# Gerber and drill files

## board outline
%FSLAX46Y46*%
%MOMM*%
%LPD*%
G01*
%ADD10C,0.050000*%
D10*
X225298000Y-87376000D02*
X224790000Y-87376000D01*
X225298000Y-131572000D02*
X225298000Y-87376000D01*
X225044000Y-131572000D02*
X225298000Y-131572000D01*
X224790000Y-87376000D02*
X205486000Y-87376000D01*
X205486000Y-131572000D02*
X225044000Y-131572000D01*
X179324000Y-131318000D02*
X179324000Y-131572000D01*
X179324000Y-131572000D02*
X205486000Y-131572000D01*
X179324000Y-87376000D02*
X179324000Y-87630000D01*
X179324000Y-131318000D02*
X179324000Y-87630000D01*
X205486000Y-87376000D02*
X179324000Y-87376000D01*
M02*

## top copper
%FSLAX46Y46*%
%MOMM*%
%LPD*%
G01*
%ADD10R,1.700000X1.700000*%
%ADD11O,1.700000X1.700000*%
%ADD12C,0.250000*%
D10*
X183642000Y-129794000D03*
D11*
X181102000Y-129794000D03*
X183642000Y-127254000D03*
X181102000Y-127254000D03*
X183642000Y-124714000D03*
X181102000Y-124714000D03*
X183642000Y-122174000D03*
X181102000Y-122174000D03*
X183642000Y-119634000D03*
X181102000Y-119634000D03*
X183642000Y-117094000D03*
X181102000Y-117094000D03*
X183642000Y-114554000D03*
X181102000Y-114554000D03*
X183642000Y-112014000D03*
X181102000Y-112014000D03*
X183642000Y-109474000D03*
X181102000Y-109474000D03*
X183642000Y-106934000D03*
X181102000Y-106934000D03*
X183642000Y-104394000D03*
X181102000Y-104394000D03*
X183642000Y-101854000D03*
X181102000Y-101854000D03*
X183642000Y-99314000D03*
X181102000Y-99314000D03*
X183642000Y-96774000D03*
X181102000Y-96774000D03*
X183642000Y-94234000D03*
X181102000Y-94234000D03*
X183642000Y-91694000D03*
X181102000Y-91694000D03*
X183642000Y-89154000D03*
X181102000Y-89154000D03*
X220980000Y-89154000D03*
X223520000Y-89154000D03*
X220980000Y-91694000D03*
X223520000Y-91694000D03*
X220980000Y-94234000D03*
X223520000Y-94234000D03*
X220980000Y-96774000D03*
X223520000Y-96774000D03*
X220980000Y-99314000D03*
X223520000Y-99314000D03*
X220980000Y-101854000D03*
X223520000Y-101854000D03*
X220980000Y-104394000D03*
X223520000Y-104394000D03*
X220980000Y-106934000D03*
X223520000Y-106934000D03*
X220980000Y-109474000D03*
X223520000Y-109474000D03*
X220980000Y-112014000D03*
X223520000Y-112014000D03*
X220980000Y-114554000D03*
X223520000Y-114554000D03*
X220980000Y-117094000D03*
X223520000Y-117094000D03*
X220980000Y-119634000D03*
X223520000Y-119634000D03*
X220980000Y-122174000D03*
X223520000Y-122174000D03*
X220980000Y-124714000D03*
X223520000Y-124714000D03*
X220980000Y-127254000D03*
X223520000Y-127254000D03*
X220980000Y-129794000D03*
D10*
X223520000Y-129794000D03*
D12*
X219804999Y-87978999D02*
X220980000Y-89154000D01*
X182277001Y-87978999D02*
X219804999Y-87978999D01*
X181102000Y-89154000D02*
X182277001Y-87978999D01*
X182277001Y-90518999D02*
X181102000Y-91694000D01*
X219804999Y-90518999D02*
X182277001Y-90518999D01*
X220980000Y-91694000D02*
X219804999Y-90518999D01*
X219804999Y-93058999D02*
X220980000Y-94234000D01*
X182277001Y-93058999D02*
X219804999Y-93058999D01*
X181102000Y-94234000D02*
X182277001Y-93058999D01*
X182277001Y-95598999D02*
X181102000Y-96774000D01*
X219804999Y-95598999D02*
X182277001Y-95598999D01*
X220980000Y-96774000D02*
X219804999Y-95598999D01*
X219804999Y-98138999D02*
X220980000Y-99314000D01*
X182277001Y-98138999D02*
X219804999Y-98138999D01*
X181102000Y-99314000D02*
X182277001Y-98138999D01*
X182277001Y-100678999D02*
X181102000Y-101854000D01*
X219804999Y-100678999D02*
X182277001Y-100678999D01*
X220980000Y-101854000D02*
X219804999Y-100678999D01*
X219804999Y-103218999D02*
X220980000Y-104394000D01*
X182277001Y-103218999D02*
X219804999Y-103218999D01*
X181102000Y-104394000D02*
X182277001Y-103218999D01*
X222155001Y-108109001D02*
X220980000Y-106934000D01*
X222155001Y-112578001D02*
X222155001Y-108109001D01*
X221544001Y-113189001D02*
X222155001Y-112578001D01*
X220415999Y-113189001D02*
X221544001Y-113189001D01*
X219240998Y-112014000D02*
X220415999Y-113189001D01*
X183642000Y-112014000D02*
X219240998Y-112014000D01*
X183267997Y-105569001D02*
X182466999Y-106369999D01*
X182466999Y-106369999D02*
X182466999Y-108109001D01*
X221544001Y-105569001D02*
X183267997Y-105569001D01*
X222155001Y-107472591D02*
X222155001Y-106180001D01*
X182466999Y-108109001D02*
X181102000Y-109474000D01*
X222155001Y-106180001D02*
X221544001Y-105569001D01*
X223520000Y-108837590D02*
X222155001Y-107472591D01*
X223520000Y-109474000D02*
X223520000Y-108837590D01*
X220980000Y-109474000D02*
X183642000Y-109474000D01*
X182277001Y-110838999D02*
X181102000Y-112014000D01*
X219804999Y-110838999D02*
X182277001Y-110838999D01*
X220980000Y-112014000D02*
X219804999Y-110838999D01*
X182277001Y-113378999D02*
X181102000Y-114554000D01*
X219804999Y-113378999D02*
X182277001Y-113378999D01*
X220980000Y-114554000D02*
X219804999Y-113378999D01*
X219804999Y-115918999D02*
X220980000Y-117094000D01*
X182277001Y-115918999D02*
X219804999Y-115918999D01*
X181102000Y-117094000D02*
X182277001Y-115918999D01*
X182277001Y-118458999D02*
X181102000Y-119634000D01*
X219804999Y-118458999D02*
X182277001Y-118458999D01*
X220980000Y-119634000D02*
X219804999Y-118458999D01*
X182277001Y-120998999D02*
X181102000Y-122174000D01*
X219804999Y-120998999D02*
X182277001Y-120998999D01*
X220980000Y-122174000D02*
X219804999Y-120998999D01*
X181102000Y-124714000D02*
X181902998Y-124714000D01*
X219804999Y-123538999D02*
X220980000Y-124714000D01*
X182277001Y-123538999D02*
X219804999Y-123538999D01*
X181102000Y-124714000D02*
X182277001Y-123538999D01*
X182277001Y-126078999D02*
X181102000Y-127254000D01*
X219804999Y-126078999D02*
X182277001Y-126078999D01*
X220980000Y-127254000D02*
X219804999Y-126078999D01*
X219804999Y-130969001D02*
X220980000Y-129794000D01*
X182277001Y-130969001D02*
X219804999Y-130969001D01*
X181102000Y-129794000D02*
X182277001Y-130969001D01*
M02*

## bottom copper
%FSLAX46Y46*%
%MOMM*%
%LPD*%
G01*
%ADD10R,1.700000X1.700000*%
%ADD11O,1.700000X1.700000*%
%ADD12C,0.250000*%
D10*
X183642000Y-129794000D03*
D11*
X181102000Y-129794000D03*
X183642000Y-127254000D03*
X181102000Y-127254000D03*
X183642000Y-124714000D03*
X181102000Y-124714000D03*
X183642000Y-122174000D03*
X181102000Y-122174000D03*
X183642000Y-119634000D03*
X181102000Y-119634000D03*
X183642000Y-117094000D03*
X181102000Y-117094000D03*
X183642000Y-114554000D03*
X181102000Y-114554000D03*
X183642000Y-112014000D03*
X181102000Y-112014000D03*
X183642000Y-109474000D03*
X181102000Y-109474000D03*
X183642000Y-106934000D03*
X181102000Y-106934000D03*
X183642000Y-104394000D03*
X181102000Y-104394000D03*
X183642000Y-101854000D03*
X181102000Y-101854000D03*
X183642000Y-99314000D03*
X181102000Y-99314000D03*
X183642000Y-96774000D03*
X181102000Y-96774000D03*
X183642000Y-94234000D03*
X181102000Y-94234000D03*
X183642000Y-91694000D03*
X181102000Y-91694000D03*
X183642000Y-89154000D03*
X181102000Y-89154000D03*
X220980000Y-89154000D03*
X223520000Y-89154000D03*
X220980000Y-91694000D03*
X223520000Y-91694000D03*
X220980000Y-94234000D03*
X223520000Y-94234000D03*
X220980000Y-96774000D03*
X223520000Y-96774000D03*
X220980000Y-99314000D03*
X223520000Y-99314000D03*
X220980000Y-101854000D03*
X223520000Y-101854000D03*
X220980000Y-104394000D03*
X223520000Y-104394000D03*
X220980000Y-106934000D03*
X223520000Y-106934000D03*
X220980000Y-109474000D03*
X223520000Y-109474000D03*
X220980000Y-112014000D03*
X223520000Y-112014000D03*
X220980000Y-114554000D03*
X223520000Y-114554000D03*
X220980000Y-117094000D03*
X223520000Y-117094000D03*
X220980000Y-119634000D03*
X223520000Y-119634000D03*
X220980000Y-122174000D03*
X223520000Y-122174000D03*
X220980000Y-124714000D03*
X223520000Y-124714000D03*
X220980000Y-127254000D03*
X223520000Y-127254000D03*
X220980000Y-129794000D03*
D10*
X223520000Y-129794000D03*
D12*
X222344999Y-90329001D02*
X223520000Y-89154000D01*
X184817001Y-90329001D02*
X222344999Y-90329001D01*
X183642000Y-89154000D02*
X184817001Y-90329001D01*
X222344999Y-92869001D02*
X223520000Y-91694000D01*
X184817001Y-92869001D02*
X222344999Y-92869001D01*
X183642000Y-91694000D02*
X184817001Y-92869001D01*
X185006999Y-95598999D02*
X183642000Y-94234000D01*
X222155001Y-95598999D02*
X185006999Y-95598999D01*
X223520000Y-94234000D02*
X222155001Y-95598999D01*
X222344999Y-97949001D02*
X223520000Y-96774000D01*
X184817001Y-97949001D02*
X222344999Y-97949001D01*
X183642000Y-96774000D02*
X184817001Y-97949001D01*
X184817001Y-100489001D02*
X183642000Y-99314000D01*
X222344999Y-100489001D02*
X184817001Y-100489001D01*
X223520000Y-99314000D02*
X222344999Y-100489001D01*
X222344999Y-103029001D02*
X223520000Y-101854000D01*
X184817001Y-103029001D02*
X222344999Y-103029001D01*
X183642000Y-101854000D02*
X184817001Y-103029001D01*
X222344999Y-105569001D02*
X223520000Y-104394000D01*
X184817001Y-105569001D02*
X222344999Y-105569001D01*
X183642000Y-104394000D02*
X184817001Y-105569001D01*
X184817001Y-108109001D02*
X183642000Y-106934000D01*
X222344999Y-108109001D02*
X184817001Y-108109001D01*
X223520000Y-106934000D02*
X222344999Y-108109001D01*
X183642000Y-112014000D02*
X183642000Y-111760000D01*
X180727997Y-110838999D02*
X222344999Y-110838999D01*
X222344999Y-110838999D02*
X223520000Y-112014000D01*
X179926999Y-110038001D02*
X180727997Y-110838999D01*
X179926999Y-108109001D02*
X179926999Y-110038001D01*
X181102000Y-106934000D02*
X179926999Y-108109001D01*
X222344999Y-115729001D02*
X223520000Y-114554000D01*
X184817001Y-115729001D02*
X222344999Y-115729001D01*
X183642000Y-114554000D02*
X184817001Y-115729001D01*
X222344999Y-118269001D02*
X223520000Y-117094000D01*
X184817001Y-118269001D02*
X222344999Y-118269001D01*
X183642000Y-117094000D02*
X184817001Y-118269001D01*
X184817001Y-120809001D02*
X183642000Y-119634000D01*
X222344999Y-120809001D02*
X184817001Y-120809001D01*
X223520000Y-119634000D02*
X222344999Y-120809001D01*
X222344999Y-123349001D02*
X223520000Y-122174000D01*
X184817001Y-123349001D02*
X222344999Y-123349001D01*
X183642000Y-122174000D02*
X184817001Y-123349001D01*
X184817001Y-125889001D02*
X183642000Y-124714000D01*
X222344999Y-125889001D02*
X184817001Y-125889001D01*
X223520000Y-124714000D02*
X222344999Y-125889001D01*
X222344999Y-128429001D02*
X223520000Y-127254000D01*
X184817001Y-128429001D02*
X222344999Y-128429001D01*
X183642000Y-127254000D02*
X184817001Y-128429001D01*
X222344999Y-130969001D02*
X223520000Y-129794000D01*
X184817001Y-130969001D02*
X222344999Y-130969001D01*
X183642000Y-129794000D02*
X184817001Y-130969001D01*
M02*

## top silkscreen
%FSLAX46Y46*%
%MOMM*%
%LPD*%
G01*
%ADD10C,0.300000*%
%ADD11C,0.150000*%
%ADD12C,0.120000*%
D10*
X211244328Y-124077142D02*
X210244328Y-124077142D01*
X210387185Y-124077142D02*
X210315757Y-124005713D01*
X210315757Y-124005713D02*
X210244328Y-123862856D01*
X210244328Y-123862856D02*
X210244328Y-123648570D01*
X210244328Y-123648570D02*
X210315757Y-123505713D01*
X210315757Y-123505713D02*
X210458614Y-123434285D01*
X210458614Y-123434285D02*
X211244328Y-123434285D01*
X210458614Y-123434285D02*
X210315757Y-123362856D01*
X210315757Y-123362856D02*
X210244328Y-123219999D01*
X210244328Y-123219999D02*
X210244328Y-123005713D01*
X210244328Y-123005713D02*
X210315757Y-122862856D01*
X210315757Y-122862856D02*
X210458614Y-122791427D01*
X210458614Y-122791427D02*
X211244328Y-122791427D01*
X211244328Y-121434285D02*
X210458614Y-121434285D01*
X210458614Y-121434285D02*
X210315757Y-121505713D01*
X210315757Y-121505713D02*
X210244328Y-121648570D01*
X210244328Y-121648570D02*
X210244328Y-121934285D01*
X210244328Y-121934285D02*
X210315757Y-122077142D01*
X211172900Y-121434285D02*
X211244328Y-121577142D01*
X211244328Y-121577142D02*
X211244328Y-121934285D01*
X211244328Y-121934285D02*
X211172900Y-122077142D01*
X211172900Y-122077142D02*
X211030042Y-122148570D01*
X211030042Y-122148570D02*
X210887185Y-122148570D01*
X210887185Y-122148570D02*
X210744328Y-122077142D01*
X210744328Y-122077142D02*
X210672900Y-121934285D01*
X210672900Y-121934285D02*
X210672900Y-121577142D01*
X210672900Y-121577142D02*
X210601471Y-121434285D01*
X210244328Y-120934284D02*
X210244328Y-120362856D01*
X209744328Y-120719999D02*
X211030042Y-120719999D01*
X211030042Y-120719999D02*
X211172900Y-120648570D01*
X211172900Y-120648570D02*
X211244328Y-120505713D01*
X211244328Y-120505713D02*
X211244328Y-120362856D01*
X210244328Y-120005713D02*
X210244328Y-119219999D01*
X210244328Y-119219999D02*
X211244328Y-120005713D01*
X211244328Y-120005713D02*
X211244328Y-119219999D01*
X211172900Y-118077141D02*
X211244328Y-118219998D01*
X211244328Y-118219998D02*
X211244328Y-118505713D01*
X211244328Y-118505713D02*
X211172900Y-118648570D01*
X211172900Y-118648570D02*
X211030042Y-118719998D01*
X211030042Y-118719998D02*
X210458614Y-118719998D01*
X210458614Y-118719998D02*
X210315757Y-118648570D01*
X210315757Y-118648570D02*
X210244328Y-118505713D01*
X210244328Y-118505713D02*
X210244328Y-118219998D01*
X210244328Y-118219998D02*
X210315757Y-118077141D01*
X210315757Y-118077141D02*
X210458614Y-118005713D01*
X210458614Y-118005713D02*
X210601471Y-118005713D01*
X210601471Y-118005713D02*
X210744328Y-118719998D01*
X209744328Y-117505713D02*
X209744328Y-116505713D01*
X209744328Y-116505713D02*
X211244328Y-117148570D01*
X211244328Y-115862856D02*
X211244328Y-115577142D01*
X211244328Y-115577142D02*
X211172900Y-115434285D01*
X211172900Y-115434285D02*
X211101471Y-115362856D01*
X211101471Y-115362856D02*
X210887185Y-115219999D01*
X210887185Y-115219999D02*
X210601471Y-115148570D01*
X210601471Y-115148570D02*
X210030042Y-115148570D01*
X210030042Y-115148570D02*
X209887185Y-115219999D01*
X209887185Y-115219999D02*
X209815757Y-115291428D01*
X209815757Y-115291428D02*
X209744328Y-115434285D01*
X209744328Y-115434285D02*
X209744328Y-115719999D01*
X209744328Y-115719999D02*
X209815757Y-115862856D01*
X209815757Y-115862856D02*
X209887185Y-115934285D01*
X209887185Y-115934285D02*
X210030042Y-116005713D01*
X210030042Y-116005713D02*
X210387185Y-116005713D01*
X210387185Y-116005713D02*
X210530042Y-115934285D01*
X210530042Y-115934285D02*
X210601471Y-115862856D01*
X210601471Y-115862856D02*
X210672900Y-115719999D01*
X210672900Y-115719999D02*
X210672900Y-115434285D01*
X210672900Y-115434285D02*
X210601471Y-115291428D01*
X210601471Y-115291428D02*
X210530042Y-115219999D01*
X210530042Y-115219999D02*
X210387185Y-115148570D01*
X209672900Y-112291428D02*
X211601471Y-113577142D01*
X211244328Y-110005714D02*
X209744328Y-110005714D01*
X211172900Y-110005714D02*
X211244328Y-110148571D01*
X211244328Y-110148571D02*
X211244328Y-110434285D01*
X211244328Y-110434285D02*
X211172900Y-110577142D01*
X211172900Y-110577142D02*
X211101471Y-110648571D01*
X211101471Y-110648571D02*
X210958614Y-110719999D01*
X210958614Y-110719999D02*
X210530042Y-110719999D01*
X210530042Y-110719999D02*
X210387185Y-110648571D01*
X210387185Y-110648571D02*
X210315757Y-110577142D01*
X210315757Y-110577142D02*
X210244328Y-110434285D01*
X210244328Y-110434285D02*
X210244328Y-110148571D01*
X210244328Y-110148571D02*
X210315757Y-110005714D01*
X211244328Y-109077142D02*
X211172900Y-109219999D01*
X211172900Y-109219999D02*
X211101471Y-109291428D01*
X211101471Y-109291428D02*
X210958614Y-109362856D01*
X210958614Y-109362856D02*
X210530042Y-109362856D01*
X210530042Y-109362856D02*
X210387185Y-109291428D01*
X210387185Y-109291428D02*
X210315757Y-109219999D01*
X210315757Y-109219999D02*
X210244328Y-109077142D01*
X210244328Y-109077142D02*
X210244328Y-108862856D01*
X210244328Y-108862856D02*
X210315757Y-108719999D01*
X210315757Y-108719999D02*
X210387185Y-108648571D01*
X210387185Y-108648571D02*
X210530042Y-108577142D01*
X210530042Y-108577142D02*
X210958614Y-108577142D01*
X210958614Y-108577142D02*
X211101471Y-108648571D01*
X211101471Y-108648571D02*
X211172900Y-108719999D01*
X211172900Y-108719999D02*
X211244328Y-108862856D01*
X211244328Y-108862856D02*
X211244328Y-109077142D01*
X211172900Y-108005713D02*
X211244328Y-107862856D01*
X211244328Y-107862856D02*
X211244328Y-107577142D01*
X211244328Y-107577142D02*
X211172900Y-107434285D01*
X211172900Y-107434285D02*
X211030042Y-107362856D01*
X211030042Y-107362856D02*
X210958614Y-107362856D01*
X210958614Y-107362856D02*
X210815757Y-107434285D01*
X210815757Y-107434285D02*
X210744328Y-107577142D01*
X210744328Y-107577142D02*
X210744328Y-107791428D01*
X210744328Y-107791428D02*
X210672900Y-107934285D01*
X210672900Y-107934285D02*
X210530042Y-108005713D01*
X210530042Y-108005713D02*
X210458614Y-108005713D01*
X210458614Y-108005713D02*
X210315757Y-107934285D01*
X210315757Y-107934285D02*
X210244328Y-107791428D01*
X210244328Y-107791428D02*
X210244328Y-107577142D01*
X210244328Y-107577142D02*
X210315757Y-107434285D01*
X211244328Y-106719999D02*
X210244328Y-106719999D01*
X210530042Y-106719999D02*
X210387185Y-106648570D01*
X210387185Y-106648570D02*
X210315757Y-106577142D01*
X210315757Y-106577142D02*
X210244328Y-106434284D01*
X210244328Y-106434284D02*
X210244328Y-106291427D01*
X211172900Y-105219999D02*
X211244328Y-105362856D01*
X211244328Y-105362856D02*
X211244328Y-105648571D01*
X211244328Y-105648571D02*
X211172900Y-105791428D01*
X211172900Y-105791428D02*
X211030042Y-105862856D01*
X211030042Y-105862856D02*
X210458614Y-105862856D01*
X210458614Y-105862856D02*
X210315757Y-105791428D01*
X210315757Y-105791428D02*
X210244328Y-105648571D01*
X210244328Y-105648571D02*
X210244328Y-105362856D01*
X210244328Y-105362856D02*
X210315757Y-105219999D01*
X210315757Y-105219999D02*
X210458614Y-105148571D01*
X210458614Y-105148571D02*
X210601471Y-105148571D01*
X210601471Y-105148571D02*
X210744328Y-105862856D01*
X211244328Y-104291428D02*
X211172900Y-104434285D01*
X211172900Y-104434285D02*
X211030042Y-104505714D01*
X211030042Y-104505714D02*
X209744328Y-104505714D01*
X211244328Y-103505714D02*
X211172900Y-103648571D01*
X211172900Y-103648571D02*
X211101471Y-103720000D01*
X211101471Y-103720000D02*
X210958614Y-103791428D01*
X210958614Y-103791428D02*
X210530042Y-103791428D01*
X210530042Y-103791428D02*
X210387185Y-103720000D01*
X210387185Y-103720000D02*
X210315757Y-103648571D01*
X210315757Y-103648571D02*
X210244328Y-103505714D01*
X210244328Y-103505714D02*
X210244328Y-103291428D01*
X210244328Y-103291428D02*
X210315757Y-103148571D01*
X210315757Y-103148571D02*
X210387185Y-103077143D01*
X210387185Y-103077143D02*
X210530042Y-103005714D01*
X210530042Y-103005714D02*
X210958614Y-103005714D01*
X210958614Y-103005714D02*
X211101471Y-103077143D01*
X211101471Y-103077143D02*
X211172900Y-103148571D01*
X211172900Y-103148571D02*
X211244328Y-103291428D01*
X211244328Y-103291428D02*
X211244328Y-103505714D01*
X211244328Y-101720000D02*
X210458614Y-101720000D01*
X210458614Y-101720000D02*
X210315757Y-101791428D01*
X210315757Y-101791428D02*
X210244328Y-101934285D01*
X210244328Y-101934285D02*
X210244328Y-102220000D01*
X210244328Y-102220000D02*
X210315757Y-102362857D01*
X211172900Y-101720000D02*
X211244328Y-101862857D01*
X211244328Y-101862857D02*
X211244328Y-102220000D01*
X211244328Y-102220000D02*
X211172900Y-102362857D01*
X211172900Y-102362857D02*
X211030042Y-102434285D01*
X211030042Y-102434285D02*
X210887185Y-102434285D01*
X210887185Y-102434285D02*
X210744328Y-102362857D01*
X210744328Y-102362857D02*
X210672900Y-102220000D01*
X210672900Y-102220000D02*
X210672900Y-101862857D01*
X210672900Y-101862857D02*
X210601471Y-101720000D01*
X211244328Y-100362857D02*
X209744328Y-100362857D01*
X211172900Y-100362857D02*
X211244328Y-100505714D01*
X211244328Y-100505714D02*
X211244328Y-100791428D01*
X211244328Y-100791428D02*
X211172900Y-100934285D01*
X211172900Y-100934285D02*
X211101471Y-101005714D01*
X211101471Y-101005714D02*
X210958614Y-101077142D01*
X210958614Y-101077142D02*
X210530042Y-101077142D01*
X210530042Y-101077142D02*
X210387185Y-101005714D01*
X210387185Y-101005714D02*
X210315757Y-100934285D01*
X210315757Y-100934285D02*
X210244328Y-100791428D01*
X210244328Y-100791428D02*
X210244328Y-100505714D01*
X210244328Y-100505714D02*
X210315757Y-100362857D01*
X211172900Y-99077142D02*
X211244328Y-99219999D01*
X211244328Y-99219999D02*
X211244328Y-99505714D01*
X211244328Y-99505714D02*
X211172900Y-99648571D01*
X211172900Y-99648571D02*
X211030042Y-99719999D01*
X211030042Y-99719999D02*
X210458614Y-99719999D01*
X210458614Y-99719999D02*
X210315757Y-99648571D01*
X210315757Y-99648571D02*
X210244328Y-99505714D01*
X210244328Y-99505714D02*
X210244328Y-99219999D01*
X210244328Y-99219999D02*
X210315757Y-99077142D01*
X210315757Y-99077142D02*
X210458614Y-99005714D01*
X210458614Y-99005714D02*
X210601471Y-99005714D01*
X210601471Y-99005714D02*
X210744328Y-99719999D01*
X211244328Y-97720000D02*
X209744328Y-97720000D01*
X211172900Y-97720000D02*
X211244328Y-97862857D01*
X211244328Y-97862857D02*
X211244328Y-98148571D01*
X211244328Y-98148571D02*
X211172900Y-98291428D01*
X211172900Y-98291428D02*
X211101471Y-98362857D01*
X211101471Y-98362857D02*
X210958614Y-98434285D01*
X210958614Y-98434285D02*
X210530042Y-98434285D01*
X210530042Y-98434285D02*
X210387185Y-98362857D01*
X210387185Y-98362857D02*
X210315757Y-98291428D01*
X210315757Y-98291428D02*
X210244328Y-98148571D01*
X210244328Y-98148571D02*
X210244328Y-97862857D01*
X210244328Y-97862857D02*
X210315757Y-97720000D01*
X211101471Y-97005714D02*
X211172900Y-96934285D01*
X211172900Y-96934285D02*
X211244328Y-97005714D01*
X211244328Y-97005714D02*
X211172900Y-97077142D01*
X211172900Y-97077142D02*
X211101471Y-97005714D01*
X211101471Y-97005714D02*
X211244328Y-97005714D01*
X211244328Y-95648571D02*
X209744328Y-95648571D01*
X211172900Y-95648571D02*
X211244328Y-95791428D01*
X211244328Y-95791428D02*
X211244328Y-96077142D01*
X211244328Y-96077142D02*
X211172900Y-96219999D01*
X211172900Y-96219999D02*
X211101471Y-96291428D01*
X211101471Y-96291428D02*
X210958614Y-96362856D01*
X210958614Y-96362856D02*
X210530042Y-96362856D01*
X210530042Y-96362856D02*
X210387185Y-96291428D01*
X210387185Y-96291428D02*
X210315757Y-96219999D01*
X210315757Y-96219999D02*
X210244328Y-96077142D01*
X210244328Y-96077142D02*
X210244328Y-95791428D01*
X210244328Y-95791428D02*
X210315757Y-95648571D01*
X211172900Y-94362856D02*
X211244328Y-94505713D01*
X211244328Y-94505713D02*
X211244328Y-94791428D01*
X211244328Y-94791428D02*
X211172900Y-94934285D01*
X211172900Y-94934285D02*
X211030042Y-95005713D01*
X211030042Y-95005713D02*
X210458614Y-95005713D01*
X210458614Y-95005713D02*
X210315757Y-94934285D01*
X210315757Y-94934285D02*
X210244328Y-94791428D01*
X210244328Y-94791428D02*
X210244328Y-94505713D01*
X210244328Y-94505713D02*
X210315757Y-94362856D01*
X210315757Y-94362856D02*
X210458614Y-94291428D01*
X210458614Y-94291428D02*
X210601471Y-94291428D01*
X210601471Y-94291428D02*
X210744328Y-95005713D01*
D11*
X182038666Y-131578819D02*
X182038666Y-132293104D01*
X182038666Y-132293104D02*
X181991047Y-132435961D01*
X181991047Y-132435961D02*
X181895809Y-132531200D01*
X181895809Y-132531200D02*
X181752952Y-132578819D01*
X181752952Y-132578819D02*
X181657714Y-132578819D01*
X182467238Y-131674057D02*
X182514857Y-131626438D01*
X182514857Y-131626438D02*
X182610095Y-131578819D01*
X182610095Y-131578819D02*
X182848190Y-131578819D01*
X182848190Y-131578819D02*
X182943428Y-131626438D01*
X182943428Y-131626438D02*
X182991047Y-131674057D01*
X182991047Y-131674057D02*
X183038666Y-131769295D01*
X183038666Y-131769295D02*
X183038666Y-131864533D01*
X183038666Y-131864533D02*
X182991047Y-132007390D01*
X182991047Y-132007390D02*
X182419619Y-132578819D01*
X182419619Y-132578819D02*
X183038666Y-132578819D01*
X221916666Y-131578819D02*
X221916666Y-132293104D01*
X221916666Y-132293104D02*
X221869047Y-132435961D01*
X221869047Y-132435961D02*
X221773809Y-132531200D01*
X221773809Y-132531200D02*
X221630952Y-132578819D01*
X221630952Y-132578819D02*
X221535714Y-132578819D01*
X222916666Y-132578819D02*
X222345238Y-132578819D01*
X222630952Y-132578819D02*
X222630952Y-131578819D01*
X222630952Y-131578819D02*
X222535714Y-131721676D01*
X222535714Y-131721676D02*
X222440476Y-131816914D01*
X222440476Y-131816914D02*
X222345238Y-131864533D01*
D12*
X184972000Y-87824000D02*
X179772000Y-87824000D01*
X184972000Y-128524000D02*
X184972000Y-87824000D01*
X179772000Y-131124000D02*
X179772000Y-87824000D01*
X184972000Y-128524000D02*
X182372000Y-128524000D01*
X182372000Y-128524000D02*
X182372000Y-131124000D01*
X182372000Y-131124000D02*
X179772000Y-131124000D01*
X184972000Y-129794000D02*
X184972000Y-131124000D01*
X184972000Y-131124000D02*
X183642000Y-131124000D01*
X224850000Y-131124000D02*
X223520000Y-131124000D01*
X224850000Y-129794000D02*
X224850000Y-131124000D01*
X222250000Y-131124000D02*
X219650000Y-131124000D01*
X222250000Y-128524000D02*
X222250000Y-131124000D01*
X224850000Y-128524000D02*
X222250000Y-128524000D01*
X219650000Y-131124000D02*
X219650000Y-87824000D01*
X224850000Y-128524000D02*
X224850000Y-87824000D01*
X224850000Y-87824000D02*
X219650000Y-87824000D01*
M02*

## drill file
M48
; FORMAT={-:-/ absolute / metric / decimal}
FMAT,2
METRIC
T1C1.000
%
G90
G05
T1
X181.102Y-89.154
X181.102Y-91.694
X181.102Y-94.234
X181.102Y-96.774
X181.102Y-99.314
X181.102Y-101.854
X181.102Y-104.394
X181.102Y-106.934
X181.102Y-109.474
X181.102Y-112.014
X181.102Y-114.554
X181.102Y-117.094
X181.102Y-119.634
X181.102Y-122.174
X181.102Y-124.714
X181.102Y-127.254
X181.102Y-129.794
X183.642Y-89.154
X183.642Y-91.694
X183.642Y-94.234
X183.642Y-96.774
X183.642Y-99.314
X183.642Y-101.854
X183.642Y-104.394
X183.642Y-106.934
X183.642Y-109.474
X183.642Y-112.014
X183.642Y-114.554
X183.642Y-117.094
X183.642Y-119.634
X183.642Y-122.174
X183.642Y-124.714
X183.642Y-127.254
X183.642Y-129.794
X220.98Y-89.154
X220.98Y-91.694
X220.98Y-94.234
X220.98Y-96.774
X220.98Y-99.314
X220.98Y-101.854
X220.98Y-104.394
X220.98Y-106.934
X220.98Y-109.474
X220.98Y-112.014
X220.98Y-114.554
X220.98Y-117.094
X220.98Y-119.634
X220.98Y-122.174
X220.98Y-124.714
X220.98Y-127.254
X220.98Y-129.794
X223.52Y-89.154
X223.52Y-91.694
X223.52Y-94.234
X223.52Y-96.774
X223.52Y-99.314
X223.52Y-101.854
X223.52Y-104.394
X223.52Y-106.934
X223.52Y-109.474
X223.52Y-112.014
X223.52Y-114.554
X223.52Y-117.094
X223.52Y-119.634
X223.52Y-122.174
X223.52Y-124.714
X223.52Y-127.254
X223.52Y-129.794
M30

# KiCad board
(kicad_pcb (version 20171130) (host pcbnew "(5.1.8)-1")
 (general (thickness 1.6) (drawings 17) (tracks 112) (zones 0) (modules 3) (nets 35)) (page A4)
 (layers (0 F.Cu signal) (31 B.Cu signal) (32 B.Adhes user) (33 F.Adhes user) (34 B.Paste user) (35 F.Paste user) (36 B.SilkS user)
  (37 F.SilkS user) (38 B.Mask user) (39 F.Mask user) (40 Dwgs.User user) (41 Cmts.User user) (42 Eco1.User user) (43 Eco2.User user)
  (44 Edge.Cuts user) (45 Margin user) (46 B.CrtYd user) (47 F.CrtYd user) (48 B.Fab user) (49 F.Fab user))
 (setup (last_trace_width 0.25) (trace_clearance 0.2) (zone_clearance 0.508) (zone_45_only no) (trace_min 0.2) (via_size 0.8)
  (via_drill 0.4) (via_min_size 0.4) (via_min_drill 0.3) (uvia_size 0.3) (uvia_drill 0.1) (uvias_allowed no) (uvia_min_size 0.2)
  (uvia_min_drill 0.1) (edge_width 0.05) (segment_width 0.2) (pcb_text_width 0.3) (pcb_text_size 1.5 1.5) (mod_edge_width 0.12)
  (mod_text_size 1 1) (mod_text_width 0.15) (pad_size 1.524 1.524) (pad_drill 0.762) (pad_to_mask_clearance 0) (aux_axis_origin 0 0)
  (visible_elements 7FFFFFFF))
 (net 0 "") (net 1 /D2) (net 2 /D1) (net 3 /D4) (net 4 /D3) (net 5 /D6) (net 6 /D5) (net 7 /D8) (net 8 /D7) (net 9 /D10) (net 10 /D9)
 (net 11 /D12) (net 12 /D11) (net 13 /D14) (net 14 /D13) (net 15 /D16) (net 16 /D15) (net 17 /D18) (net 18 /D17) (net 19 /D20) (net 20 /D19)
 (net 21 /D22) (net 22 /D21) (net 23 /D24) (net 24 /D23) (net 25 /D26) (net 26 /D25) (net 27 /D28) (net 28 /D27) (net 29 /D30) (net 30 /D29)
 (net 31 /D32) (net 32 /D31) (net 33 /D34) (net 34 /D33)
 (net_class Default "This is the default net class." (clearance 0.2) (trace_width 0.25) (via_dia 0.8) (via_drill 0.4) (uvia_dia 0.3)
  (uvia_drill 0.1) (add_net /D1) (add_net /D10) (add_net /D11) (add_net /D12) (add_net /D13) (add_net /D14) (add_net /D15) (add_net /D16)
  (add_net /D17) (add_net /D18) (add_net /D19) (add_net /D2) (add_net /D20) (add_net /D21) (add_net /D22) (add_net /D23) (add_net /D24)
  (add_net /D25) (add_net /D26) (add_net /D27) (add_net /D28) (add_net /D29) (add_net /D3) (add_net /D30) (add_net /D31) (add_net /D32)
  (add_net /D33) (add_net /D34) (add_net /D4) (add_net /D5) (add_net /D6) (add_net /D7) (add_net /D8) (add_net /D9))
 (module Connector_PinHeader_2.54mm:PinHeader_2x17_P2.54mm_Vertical (layer F.Cu) (at 183.642 129.794 180)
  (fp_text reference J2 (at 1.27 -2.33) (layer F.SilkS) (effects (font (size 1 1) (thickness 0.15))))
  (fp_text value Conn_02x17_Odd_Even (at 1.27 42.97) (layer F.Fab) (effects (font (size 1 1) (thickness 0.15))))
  (fp_line (start -1.33 41.97) (end 3.87 41.97) (layer F.SilkS) (width 0.12))
  (fp_line (start -1.33 1.27) (end -1.33 41.97) (layer F.SilkS) (width 0.12))
  (fp_line (start 3.87 -1.33) (end 3.87 41.97) (layer F.SilkS) (width 0.12))
  (fp_line (start -1.33 1.27) (end 1.27 1.27) (layer F.SilkS) (width 0.12))
  (fp_line (start 1.27 1.27) (end 1.27 -1.33) (layer F.SilkS) (width 0.12))
  (fp_line (start 1.27 -1.33) (end 3.87 -1.33) (layer F.SilkS) (width 0.12))
  (fp_line (start -1.33 0) (end -1.33 -1.33) (layer F.SilkS) (width 0.12))
  (fp_line (start -1.33 -1.33) (end 0 -1.33) (layer F.SilkS) (width 0.12))
  (pad 1 thru_hole rect (at 0 0 180) (size 1.7 1.7) (drill 1) (layers *.Cu *.Mask) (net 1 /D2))
  (pad 2 thru_hole oval (at 2.54 0 180) (size 1.7 1.7) (drill 1) (layers *.Cu *.Mask) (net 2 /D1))
  (pad 3 thru_hole oval (at 0 2.54 180) (size 1.7 1.7) (drill 1) (layers *.Cu *.Mask) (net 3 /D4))
  (pad 4 thru_hole oval (at 2.54 2.54 180) (size 1.7 1.7) (drill 1) (layers *.Cu *.Mask) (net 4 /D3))
  (pad 5 thru_hole oval (at 0 5.08 180) (size 1.7 1.7) (drill 1) (layers *.Cu *.Mask) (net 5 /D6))
  (pad 6 thru_hole oval (at 2.54 5.08 180) (size 1.7 1.7) (drill 1) (layers *.Cu *.Mask) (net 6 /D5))
  (pad 7 thru_hole oval (at 0 7.62 180) (size 1.7 1.7) (drill 1) (layers *.Cu *.Mask) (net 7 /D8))
  (pad 8 thru_hole oval (at 2.54 7.62 180) (size 1.7 1.7) (drill 1) (layers *.Cu *.Mask) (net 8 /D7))
  (pad 9 thru_hole oval (at 0 10.16 180) (size 1.7 1.7) (drill 1) (layers *.Cu *.Mask) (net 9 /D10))
  (pad 10 thru_hole oval (at 2.54 10.16 180) (size 1.7 1.7) (drill 1) (layers *.Cu *.Mask) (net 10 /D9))
  (pad 11 thru_hole oval (at 0 12.7 180) (size 1.7 1.7) (drill 1) (layers *.Cu *.Mask) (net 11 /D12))
  (pad 12 thru_hole oval (at 2.54 12.7 180) (size 1.7 1.7) (drill 1) (layers *.Cu *.Mask) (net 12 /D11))
  (pad 13 thru_hole oval (at 0 15.24 180) (size 1.7 1.7) (drill 1) (layers *.Cu *.Mask) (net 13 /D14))
  (pad 14 thru_hole oval (at 2.54 15.24 180) (size 1.7 1.7) (drill 1) (layers *.Cu *.Mask) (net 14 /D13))
  (pad 15 thru_hole oval (at 0 17.78 180) (size 1.7 1.7) (drill 1) (layers *.Cu *.Mask) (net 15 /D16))
  (pad 16 thru_hole oval (at 2.54 17.78 180) (size 1.7 1.7) (drill 1) (layers *.Cu *.Mask) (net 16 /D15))
  (pad 17 thru_hole oval (at 0 20.32 180) (size 1.7 1.7) (drill 1) (layers *.Cu *.Mask) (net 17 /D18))
  (pad 18 thru_hole oval (at 2.54 20.32 180) (size 1.7 1.7) (drill 1) (layers *.Cu *.Mask) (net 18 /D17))
  (pad 19 thru_hole oval (at 0 22.86 180) (size 1.7 1.7) (drill 1) (layers *.Cu *.Mask) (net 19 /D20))
  (pad 20 thru_hole oval (at 2.54 22.86 180) (size 1.7 1.7) (drill 1) (layers *.Cu *.Mask) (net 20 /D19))
  (pad 21 thru_hole oval (at 0 25.4 180) (size 1.7 1.7) (drill 1) (layers *.Cu *.Mask) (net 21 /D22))
  (pad 22 thru_hole oval (at 2.54 25.4 180) (size 1.7 1.7) (drill 1) (layers *.Cu *.Mask) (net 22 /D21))
  (pad 23 thru_hole oval (at 0 27.94 180) (size 1.7 1.7) (drill 1) (layers *.Cu *.Mask) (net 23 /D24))
  (pad 24 thru_hole oval (at 2.54 27.94 180) (size 1.7 1.7) (drill 1) (layers *.Cu *.Mask) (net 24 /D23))
  (pad 25 thru_hole oval (at 0 30.48 180) (size 1.7 1.7) (drill 1) (layers *.Cu *.Mask) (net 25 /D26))
  (pad 26 thru_hole oval (at 2.54 30.48 180) (size 1.7 1.7) (drill 1) (layers *.Cu *.Mask) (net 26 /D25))
  (pad 27 thru_hole oval (at 0 33.02 180) (size 1.7 1.7) (drill 1) (layers *.Cu *.Mask) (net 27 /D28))
  (pad 28 thru_hole oval (at 2.54 33.02 180) (size 1.7 1.7) (drill 1) (layers *.Cu *.Mask) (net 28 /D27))
  (pad 29 thru_hole oval (at 0 35.56 180) (size 1.7 1.7) (drill 1) (layers *.Cu *.Mask) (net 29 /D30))
  (pad 30 thru_hole oval (at 2.54 35.56 180) (size 1.7 1.7) (drill 1) (layers *.Cu *.Mask) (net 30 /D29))
  (pad 31 thru_hole oval (at 0 38.1 180) (size 1.7 1.7) (drill 1) (layers *.Cu *.Mask) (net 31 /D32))
  (pad 32 thru_hole oval (at 2.54 38.1 180) (size 1.7 1.7) (drill 1) (layers *.Cu *.Mask) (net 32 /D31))
  (pad 33 thru_hole oval (at 0 40.64 180) (size 1.7 1.7) (drill 1) (layers *.Cu *.Mask) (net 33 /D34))
  (pad 34 thru_hole oval (at 2.54 40.64 180) (size 1.7 1.7) (drill 1) (layers *.Cu *.Mask) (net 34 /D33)))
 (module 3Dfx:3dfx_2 (layer B.Cu) (at 201.422 109.982 270)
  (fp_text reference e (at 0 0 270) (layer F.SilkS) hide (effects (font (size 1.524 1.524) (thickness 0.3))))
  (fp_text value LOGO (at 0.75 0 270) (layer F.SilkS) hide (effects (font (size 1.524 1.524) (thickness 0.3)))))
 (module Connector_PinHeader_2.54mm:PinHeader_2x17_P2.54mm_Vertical (layer F.Cu) (at 223.52 129.794 180)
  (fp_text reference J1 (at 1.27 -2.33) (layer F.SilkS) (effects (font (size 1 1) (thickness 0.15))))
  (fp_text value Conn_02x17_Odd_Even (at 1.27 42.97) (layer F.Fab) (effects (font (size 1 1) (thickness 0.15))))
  (fp_line (start -1.33 -1.33) (end 0 -1.33) (layer F.SilkS) (width 0.12))
  (fp_line (start -1.33 0) (end -1.33 -1.33) (layer F.SilkS) (width 0.12))
  (fp_line (start 1.27 -1.33) (end 3.87 -1.33) (layer F.SilkS) (width 0.12))
  (fp_line (start 1.27 1.27) (end 1.27 -1.33) (layer F.SilkS) (width 0.12))
  (fp_line (start -1.33 1.27) (end 1.27 1.27) (layer F.SilkS) (width 0.12))
  (fp_line (start 3.87 -1.33) (end 3.87 41.97) (layer F.SilkS) (width 0.12))
  (fp_line (start -1.33 1.27) (end -1.33 41.97) (layer F.SilkS) (width 0.12))
  (fp_line (start -1.33 41.97) (end 3.87 41.97) (layer F.SilkS) (width 0.12))
  (pad 34 thru_hole oval (at 2.54 40.64 180) (size 1.7 1.7) (drill 1) (layers *.Cu *.Mask) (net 34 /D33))
  (pad 33 thru_hole oval (at 0 40.64 180) (size 1.7 1.7) (drill 1) (layers *.Cu *.Mask) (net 33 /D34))
  (pad 32 thru_hole oval (at 2.54 38.1 180) (size 1.7 1.7) (drill 1) (layers *.Cu *.Mask) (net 32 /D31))
  (pad 31 thru_hole oval (at 0 38.1 180) (size 1.7 1.7) (drill 1) (layers *.Cu *.Mask) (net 31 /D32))
  (pad 30 thru_hole oval (at 2.54 35.56 180) (size 1.7 1.7) (drill 1) (layers *.Cu *.Mask) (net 30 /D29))
  (pad 29 thru_hole oval (at 0 35.56 180) (size 1.7 1.7) (drill 1) (layers *.Cu *.Mask) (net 29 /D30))
  (pad 28 thru_hole oval (at 2.54 33.02 180) (size 1.7 1.7) (drill 1) (layers *.Cu *.Mask) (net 28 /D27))
  (pad 27 thru_hole oval (at 0 33.02 180) (size 1.7 1.7) (drill 1) (layers *.Cu *.Mask) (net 27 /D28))
  (pad 26 thru_hole oval (at 2.54 30.48 180) (size 1.7 1.7) (drill 1) (layers *.Cu *.Mask) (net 26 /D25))
  (pad 25 thru_hole oval (at 0 30.48 180) (size 1.7 1.7) (drill 1) (layers *.Cu *.Mask) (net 25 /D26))
  (pad 24 thru_hole oval (at 2.54 27.94 180) (size 1.7 1.7) (drill 1) (layers *.Cu *.Mask) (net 24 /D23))
  (pad 23 thru_hole oval (at 0 27.94 180) (size 1.7 1.7) (drill 1) (layers *.Cu *.Mask) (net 23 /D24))
  (pad 22 thru_hole oval (at 2.54 25.4 180) (size 1.7 1.7) (drill 1) (layers *.Cu *.Mask) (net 22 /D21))
  (pad 21 thru_hole oval (at 0 25.4 180) (size 1.7 1.7) (drill 1) (layers *.Cu *.Mask) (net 21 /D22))
  (pad 20 thru_hole oval (at 2.54 22.86 180) (size 1.7 1.7) (drill 1) (layers *.Cu *.Mask) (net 15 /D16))
  (pad 19 thru_hole oval (at 0 22.86 180) (size 1.7 1.7) (drill 1) (layers *.Cu *.Mask) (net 19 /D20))
  (pad 18 thru_hole oval (at 2.54 20.32 180) (size 1.7 1.7) (drill 1) (layers *.Cu *.Mask) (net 17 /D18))
  (pad 17 thru_hole oval (at 0 20.32 180) (size 1.7 1.7) (drill 1) (layers *.Cu *.Mask) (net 18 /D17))
  (pad 16 thru_hole oval (at 2.54 17.78 180) (size 1.7 1.7) (drill 1) (layers *.Cu *.Mask) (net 16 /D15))
  (pad 15 thru_hole oval (at 0 17.78 180) (size 1.7 1.7) (drill 1) (layers *.Cu *.Mask) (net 20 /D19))
  (pad 14 thru_hole oval (at 2.54 15.24 180) (size 1.7 1.7) (drill 1) (layers *.Cu *.Mask) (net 14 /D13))
  (pad 13 thru_hole oval (at 0 15.24 180) (size 1.7 1.7) (drill 1) (layers *.Cu *.Mask) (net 13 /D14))
  (pad 12 thru_hole oval (at 2.54 12.7 180) (size 1.7 1.7) (drill 1) (layers *.Cu *.Mask) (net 12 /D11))
  (pad 11 thru_hole oval (at 0 12.7 180) (size 1.7 1.7) (drill 1) (layers *.Cu *.Mask) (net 11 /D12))
  (pad 10 thru_hole oval (at 2.54 10.16 180) (size 1.7 1.7) (drill 1) (layers *.Cu *.Mask) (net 10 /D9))
  (pad 9 thru_hole oval (at 0 10.16 180) (size 1.7 1.7) (drill 1) (layers *.Cu *.Mask) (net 9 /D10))
  (pad 8 thru_hole oval (at 2.54 7.62 180) (size 1.7 1.7) (drill 1) (layers *.Cu *.Mask) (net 8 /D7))
  (pad 7 thru_hole oval (at 0 7.62 180) (size 1.7 1.7) (drill 1) (layers *.Cu *.Mask) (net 7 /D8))
  (pad 6 thru_hole oval (at 2.54 5.08 180) (size 1.7 1.7) (drill 1) (layers *.Cu *.Mask) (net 6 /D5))
  (pad 5 thru_hole oval (at 0 5.08 180) (size 1.7 1.7) (drill 1) (layers *.Cu *.Mask) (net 5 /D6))
  (pad 4 thru_hole oval (at 2.54 2.54 180) (size 1.7 1.7) (drill 1) (layers *.Cu *.Mask) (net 4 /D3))
  (pad 3 thru_hole oval (at 0 2.54 180) (size 1.7 1.7) (drill 1) (layers *.Cu *.Mask) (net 3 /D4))
  (pad 2 thru_hole oval (at 2.54 0 180) (size 1.7 1.7) (drill 1) (layers *.Cu *.Mask) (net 2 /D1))
  (pad 1 thru_hole rect (at 0 0 180) (size 1.7 1.7) (drill 1) (layers *.Cu *.Mask) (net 1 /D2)))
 (gr_line (start 225.298 87.376) (end 224.79 87.376) (layer Edge.Cuts) (width 0.05))
 (gr_line (start 225.298 131.572) (end 225.298 87.376) (layer Edge.Cuts) (width 0.05))
 (gr_line (start 225.044 131.572) (end 225.298 131.572) (layer Edge.Cuts) (width 0.05))
 (gr_line (start 224.79 87.376) (end 205.486 87.376) (layer Edge.Cuts) (width 0.05))
 (gr_line (start 205.486 131.572) (end 225.044 131.572) (layer Edge.Cuts) (width 0.05))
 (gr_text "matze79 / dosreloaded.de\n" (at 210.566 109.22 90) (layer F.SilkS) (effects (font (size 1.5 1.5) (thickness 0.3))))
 (gr_line (start 179.324 131.318) (end 179.324 131.572) (layer Edge.Cuts) (width 0.05))
 (gr_line (start 179.324 131.572) (end 205.486 131.572) (layer Edge.Cuts) (width 0.05))
 (gr_line (start 179.324 87.376) (end 179.324 87.63) (layer Edge.Cuts) (width 0.05))
 (gr_line (start 179.324 131.318) (end 179.324 87.63) (layer Edge.Cuts) (width 0.05))
 (gr_line (start 205.486 87.376) (end 179.324 87.376) (layer Edge.Cuts) (width 0.05))
 (segment (start 222.344999 90.329001) (end 223.52 89.154) (width 0.25) (layer B.Cu) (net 33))
 (segment (start 184.817001 90.329001) (end 222.344999 90.329001) (width 0.25) (layer B.Cu) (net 33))
 (segment (start 183.642 89.154) (end 184.817001 90.329001) (width 0.25) (layer B.Cu) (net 33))
 (segment (start 219.804999 87.978999) (end 220.98 89.154) (width 0.25) (layer F.Cu) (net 34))
 (segment (start 182.277001 87.978999) (end 219.804999 87.978999) (width 0.25) (layer F.Cu) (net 34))
 (segment (start 181.102 89.154) (end 182.277001 87.978999) (width 0.25) (layer F.Cu) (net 34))
 (segment (start 222.344999 92.869001) (end 223.52 91.694) (width 0.25) (layer B.Cu) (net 31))
 (segment (start 184.817001 92.869001) (end 222.344999 92.869001) (width 0.25) (layer B.Cu) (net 31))
 (segment (start 183.642 91.694) (end 184.817001 92.869001) (width 0.25) (layer B.Cu) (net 31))
 (segment (start 182.277001 90.518999) (end 181.102 91.694) (width 0.25) (layer F.Cu) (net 32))
 (segment (start 219.804999 90.518999) (end 182.277001 90.518999) (width 0.25) (layer F.Cu) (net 32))
 (segment (start 220.98 91.694) (end 219.804999 90.518999) (width 0.25) (layer F.Cu) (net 32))
 (segment (start 185.006999 95.598999) (end 183.642 94.234) (width 0.25) (layer B.Cu) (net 29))
 (segment (start 222.155001 95.598999) (end 185.006999 95.598999) (width 0.25) (layer B.Cu) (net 29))
 (segment (start 223.52 94.234) (end 222.155001 95.598999) (width 0.25) (layer B.Cu) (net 29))
 (segment (start 219.804999 93.058999) (end 220.98 94.234) (width 0.25) (layer F.Cu) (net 30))
 (segment (start 182.277001 93.058999) (end 219.804999 93.058999) (width 0.25) (layer F.Cu) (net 30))
 (segment (start 181.102 94.234) (end 182.277001 93.058999) (width 0.25) (layer F.Cu) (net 30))
 (segment (start 222.344999 97.949001) (end 223.52 96.774) (width 0.25) (layer B.Cu) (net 27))
 (segment (start 184.817001 97.949001) (end 222.344999 97.949001) (width 0.25) (layer B.Cu) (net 27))
 (segment (start 183.642 96.774) (end 184.817001 97.949001) (width 0.25) (layer B.Cu) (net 27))
 (segment (start 182.277001 95.598999) (end 181.102 96.774) (width 0.25) (layer F.Cu) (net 28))
 (segment (start 219.804999 95.598999) (end 182.277001 95.598999) (width 0.25) (layer F.Cu) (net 28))
 (segment (start 220.98 96.774) (end 219.804999 95.598999) (width 0.25) (layer F.Cu) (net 28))
 (segment (start 184.817001 100.489001) (end 183.642 99.314) (width 0.25) (layer B.Cu) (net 25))
 (segment (start 222.344999 100.489001) (end 184.817001 100.489001) (width 0.25) (layer B.Cu) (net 25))
 (segment (start 223.52 99.314) (end 222.344999 100.489001) (width 0.25) (layer B.Cu) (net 25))
 (segment (start 219.804999 98.138999) (end 220.98 99.314) (width 0.25) (layer F.Cu) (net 26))
 (segment (start 182.277001 98.138999) (end 219.804999 98.138999) (width 0.25) (layer F.Cu) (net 26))
 (segment (start 181.102 99.314) (end 182.277001 98.138999) (width 0.25) (layer F.Cu) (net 26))
 (segment (start 222.344999 103.029001) (end 223.52 101.854) (width 0.25) (layer B.Cu) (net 23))
 (segment (start 184.817001 103.029001) (end 222.344999 103.029001) (width 0.25) (layer B.Cu) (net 23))
 (segment (start 183.642 101.854) (end 184.817001 103.029001) (width 0.25) (layer B.Cu) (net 23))
 (segment (start 182.277001 100.678999) (end 181.102 101.854) (width 0.25) (layer F.Cu) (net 24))
 (segment (start 219.804999 100.678999) (end 182.277001 100.678999) (width 0.25) (layer F.Cu) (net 24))
 (segment (start 220.98 101.854) (end 219.804999 100.678999) (width 0.25) (layer F.Cu) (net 24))
 (segment (start 222.344999 105.569001) (end 223.52 104.394) (width 0.25) (layer B.Cu) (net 21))
 (segment (start 184.817001 105.569001) (end 222.344999 105.569001) (width 0.25) (layer B.Cu) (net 21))
 (segment (start 183.642 104.394) (end 184.817001 105.569001) (width 0.25) (layer B.Cu) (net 21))
 (segment (start 219.804999 103.218999) (end 220.98 104.394) (width 0.25) (layer F.Cu) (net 22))
 (segment (start 182.277001 103.218999) (end 219.804999 103.218999) (width 0.25) (layer F.Cu) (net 22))
 (segment (start 181.102 104.394) (end 182.277001 103.218999) (width 0.25) (layer F.Cu) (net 22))
 (segment (start 184.817001 108.109001) (end 183.642 106.934) (width 0.25) (layer B.Cu) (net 19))
 (segment (start 222.344999 108.109001) (end 184.817001 108.109001) (width 0.25) (layer B.Cu) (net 19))
 (segment (start 223.52 106.934) (end 222.344999 108.109001) (width 0.25) (layer B.Cu) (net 19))
 (segment (start 183.642 112.014) (end 183.642 111.76) (width 0.25) (layer B.Cu) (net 15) (status 30))
 (segment (start 222.155001 108.109001) (end 220.98 106.934) (width 0.25) (layer F.Cu) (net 15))
 (segment (start 222.155001 112.578001) (end 222.155001 108.109001) (width 0.25) (layer F.Cu) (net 15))
 (segment (start 221.544001 113.189001) (end 222.155001 112.578001) (width 0.25) (layer F.Cu) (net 15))
 (segment (start 220.415999 113.189001) (end 221.544001 113.189001) (width 0.25) (layer F.Cu) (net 15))
 (segment (start 219.240998 112.014) (end 220.415999 113.189001) (width 0.25) (layer F.Cu) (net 15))
 (segment (start 183.642 112.014) (end 219.240998 112.014) (width 0.25) (layer F.Cu) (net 15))
 (segment (start 183.267997 105.569001) (end 182.466999 106.369999) (width 0.25) (layer F.Cu) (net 18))
 (segment (start 182.466999 106.369999) (end 182.466999 108.109001) (width 0.25) (layer F.Cu) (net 18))
 (segment (start 221.544001 105.569001) (end 183.267997 105.569001) (width 0.25) (layer F.Cu) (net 18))
 (segment (start 222.155001 107.472591) (end 222.155001 106.180001) (width 0.25) (layer F.Cu) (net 18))
 (segment (start 182.466999 108.109001) (end 181.102 109.474) (width 0.25) (layer F.Cu) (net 18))
 (segment (start 222.155001 106.180001) (end 221.544001 105.569001) (width 0.25) (layer F.Cu) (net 18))
 (segment (start 223.52 108.83759) (end 222.155001 107.472591) (width 0.25) (layer F.Cu) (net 18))
 (segment (start 223.52 109.474) (end 223.52 108.83759) (width 0.25) (layer F.Cu) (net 18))
 (segment (start 220.98 109.474) (end 183.642 109.474) (width 0.25) (layer F.Cu) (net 17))
 (segment (start 180.727997 110.838999) (end 222.344999 110.838999) (width 0.25) (layer B.Cu) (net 20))
 (segment (start 222.344999 110.838999) (end 223.52 112.014) (width 0.25) (layer B.Cu) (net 20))
 (segment (start 179.926999 110.038001) (end 180.727997 110.838999) (width 0.25) (layer B.Cu) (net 20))
 (segment (start 179.926999 108.109001) (end 179.926999 110.038001) (width 0.25) (layer B.Cu) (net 20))
 (segment (start 181.102 106.934) (end 179.926999 108.109001) (width 0.25) (layer B.Cu) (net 20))
 (segment (start 182.277001 110.838999) (end 181.102 112.014) (width 0.25) (layer F.Cu) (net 16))
 (segment (start 219.804999 110.838999) (end 182.277001 110.838999) (width 0.25) (layer F.Cu) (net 16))
 (segment (start 220.98 112.014) (end 219.804999 110.838999) (width 0.25) (layer F.Cu) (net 16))
 (segment (start 222.344999 115.729001) (end 223.52 114.554) (width 0.25) (layer B.Cu) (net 13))
 (segment (start 184.817001 115.729001) (end 222.344999 115.729001) (width 0.25) (layer B.Cu) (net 13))
 (segment (start 183.642 114.554) (end 184.817001 115.729001) (width 0.25) (layer B.Cu) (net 13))
 (segment (start 182.277001 113.378999) (end 181.102 114.554) (width 0.25) (layer F.Cu) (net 14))
 (segment (start 219.804999 113.378999) (end 182.277001 113.378999) (width 0.25) (layer F.Cu) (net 14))
 (segment (start 220.98 114.554) (end 219.804999 113.378999) (width 0.25) (layer F.Cu) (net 14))
 (segment (start 222.344999 118.269001) (end 223.52 117.094) (width 0.25) (layer B.Cu) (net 11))
 (segment (start 184.817001 118.269001) (end 222.344999 118.269001) (width 0.25) (layer B.Cu) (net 11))
 (segment (start 183.642 117.094) (end 184.817001 118.269001) (width 0.25) (layer B.Cu) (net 11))
 (segment (start 219.804999 115.918999) (end 220.98 117.094) (width 0.25) (layer F.Cu) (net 12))
 (segment (start 182.277001 115.918999) (end 219.804999 115.918999) (width 0.25) (layer F.Cu) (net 12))
 (segment (start 181.102 117.094) (end 182.277001 115.918999) (width 0.25) (layer F.Cu) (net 12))
 (segment (start 184.817001 120.809001) (end 183.642 119.634) (width 0.25) (layer B.Cu) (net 9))
 (segment (start 222.344999 120.809001) (end 184.817001 120.809001) (width 0.25) (layer B.Cu) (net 9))
 (segment (start 223.52 119.634) (end 222.344999 120.809001) (width 0.25) (layer B.Cu) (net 9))
 (segment (start 182.277001 118.458999) (end 181.102 119.634) (width 0.25) (layer F.Cu) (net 10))
 (segment (start 219.804999 118.458999) (end 182.277001 118.458999) (width 0.25) (layer F.Cu) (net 10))
 (segment (start 220.98 119.634) (end 219.804999 118.458999) (width 0.25) (layer F.Cu) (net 10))
 (segment (start 222.344999 123.349001) (end 223.52 122.174) (width 0.25) (layer B.Cu) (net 7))
 (segment (start 184.817001 123.349001) (end 222.344999 123.349001) (width 0.25) (layer B.Cu) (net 7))
 (segment (start 183.642 122.174) (end 184.817001 123.349001) (width 0.25) (layer B.Cu) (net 7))
 (segment (start 182.277001 120.998999) (end 181.102 122.174) (width 0.25) (layer F.Cu) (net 8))
 (segment (start 219.804999 120.998999) (end 182.277001 120.998999) (width 0.25) (layer F.Cu) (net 8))
 (segment (start 220.98 122.174) (end 219.804999 120.998999) (width 0.25) (layer F.Cu) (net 8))
 (segment (start 184.817001 125.889001) (end 183.642 124.714) (width 0.25) (layer B.Cu) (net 5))
 (segment (start 222.344999 125.889001) (end 184.817001 125.889001) (width 0.25) (layer B.Cu) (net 5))
 (segment (start 223.52 124.714) (end 222.344999 125.889001) (width 0.25) (layer B.Cu) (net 5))
 (segment (start 181.102 124.714) (end 181.902998 124.714) (width 0.25) (layer F.Cu) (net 6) (status 30))
 (segment (start 219.804999 123.538999) (end 220.98 124.714) (width 0.25) (layer F.Cu) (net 6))
 (segment (start 182.277001 123.538999) (end 219.804999 123.538999) (width 0.25) (layer F.Cu) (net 6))
 (segment (start 181.102 124.714) (end 182.277001 123.538999) (width 0.25) (layer F.Cu) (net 6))
 (segment (start 222.344999 128.429001) (end 223.52 127.254) (width 0.25) (layer B.Cu) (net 3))
 (segment (start 184.817001 128.429001) (end 222.344999 128.429001) (width 0.25) (layer B.Cu) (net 3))
 (segment (start 183.642 127.254) (end 184.817001 128.429001) (width 0.25) (layer B.Cu) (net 3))
 (segment (start 182.277001 126.078999) (end 181.102 127.254) (width 0.25) (layer F.Cu) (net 4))
 (segment (start 219.804999 126.078999) (end 182.277001 126.078999) (width 0.25) (layer F.Cu) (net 4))
 (segment (start 220.98 127.254) (end 219.804999 126.078999) (width 0.25) (layer F.Cu) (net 4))
 (segment (start 222.344999 130.969001) (end 223.52 129.794) (width 0.25) (layer B.Cu) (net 1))
 (segment (start 184.817001 130.969001) (end 222.344999 130.969001) (width 0.25) (layer B.Cu) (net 1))
 (segment (start 183.642 129.794) (end 184.817001 130.969001) (width 0.25) (layer B.Cu) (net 1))
 (segment (start 219.804999 130.969001) (end 220.98 129.794) (width 0.25) (layer F.Cu) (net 2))
 (segment (start 182.277001 130.969001) (end 219.804999 130.969001) (width 0.25) (layer F.Cu) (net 2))
 (segment (start 181.102 129.794) (end 182.277001 130.969001) (width 0.25) (layer F.Cu) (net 2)))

